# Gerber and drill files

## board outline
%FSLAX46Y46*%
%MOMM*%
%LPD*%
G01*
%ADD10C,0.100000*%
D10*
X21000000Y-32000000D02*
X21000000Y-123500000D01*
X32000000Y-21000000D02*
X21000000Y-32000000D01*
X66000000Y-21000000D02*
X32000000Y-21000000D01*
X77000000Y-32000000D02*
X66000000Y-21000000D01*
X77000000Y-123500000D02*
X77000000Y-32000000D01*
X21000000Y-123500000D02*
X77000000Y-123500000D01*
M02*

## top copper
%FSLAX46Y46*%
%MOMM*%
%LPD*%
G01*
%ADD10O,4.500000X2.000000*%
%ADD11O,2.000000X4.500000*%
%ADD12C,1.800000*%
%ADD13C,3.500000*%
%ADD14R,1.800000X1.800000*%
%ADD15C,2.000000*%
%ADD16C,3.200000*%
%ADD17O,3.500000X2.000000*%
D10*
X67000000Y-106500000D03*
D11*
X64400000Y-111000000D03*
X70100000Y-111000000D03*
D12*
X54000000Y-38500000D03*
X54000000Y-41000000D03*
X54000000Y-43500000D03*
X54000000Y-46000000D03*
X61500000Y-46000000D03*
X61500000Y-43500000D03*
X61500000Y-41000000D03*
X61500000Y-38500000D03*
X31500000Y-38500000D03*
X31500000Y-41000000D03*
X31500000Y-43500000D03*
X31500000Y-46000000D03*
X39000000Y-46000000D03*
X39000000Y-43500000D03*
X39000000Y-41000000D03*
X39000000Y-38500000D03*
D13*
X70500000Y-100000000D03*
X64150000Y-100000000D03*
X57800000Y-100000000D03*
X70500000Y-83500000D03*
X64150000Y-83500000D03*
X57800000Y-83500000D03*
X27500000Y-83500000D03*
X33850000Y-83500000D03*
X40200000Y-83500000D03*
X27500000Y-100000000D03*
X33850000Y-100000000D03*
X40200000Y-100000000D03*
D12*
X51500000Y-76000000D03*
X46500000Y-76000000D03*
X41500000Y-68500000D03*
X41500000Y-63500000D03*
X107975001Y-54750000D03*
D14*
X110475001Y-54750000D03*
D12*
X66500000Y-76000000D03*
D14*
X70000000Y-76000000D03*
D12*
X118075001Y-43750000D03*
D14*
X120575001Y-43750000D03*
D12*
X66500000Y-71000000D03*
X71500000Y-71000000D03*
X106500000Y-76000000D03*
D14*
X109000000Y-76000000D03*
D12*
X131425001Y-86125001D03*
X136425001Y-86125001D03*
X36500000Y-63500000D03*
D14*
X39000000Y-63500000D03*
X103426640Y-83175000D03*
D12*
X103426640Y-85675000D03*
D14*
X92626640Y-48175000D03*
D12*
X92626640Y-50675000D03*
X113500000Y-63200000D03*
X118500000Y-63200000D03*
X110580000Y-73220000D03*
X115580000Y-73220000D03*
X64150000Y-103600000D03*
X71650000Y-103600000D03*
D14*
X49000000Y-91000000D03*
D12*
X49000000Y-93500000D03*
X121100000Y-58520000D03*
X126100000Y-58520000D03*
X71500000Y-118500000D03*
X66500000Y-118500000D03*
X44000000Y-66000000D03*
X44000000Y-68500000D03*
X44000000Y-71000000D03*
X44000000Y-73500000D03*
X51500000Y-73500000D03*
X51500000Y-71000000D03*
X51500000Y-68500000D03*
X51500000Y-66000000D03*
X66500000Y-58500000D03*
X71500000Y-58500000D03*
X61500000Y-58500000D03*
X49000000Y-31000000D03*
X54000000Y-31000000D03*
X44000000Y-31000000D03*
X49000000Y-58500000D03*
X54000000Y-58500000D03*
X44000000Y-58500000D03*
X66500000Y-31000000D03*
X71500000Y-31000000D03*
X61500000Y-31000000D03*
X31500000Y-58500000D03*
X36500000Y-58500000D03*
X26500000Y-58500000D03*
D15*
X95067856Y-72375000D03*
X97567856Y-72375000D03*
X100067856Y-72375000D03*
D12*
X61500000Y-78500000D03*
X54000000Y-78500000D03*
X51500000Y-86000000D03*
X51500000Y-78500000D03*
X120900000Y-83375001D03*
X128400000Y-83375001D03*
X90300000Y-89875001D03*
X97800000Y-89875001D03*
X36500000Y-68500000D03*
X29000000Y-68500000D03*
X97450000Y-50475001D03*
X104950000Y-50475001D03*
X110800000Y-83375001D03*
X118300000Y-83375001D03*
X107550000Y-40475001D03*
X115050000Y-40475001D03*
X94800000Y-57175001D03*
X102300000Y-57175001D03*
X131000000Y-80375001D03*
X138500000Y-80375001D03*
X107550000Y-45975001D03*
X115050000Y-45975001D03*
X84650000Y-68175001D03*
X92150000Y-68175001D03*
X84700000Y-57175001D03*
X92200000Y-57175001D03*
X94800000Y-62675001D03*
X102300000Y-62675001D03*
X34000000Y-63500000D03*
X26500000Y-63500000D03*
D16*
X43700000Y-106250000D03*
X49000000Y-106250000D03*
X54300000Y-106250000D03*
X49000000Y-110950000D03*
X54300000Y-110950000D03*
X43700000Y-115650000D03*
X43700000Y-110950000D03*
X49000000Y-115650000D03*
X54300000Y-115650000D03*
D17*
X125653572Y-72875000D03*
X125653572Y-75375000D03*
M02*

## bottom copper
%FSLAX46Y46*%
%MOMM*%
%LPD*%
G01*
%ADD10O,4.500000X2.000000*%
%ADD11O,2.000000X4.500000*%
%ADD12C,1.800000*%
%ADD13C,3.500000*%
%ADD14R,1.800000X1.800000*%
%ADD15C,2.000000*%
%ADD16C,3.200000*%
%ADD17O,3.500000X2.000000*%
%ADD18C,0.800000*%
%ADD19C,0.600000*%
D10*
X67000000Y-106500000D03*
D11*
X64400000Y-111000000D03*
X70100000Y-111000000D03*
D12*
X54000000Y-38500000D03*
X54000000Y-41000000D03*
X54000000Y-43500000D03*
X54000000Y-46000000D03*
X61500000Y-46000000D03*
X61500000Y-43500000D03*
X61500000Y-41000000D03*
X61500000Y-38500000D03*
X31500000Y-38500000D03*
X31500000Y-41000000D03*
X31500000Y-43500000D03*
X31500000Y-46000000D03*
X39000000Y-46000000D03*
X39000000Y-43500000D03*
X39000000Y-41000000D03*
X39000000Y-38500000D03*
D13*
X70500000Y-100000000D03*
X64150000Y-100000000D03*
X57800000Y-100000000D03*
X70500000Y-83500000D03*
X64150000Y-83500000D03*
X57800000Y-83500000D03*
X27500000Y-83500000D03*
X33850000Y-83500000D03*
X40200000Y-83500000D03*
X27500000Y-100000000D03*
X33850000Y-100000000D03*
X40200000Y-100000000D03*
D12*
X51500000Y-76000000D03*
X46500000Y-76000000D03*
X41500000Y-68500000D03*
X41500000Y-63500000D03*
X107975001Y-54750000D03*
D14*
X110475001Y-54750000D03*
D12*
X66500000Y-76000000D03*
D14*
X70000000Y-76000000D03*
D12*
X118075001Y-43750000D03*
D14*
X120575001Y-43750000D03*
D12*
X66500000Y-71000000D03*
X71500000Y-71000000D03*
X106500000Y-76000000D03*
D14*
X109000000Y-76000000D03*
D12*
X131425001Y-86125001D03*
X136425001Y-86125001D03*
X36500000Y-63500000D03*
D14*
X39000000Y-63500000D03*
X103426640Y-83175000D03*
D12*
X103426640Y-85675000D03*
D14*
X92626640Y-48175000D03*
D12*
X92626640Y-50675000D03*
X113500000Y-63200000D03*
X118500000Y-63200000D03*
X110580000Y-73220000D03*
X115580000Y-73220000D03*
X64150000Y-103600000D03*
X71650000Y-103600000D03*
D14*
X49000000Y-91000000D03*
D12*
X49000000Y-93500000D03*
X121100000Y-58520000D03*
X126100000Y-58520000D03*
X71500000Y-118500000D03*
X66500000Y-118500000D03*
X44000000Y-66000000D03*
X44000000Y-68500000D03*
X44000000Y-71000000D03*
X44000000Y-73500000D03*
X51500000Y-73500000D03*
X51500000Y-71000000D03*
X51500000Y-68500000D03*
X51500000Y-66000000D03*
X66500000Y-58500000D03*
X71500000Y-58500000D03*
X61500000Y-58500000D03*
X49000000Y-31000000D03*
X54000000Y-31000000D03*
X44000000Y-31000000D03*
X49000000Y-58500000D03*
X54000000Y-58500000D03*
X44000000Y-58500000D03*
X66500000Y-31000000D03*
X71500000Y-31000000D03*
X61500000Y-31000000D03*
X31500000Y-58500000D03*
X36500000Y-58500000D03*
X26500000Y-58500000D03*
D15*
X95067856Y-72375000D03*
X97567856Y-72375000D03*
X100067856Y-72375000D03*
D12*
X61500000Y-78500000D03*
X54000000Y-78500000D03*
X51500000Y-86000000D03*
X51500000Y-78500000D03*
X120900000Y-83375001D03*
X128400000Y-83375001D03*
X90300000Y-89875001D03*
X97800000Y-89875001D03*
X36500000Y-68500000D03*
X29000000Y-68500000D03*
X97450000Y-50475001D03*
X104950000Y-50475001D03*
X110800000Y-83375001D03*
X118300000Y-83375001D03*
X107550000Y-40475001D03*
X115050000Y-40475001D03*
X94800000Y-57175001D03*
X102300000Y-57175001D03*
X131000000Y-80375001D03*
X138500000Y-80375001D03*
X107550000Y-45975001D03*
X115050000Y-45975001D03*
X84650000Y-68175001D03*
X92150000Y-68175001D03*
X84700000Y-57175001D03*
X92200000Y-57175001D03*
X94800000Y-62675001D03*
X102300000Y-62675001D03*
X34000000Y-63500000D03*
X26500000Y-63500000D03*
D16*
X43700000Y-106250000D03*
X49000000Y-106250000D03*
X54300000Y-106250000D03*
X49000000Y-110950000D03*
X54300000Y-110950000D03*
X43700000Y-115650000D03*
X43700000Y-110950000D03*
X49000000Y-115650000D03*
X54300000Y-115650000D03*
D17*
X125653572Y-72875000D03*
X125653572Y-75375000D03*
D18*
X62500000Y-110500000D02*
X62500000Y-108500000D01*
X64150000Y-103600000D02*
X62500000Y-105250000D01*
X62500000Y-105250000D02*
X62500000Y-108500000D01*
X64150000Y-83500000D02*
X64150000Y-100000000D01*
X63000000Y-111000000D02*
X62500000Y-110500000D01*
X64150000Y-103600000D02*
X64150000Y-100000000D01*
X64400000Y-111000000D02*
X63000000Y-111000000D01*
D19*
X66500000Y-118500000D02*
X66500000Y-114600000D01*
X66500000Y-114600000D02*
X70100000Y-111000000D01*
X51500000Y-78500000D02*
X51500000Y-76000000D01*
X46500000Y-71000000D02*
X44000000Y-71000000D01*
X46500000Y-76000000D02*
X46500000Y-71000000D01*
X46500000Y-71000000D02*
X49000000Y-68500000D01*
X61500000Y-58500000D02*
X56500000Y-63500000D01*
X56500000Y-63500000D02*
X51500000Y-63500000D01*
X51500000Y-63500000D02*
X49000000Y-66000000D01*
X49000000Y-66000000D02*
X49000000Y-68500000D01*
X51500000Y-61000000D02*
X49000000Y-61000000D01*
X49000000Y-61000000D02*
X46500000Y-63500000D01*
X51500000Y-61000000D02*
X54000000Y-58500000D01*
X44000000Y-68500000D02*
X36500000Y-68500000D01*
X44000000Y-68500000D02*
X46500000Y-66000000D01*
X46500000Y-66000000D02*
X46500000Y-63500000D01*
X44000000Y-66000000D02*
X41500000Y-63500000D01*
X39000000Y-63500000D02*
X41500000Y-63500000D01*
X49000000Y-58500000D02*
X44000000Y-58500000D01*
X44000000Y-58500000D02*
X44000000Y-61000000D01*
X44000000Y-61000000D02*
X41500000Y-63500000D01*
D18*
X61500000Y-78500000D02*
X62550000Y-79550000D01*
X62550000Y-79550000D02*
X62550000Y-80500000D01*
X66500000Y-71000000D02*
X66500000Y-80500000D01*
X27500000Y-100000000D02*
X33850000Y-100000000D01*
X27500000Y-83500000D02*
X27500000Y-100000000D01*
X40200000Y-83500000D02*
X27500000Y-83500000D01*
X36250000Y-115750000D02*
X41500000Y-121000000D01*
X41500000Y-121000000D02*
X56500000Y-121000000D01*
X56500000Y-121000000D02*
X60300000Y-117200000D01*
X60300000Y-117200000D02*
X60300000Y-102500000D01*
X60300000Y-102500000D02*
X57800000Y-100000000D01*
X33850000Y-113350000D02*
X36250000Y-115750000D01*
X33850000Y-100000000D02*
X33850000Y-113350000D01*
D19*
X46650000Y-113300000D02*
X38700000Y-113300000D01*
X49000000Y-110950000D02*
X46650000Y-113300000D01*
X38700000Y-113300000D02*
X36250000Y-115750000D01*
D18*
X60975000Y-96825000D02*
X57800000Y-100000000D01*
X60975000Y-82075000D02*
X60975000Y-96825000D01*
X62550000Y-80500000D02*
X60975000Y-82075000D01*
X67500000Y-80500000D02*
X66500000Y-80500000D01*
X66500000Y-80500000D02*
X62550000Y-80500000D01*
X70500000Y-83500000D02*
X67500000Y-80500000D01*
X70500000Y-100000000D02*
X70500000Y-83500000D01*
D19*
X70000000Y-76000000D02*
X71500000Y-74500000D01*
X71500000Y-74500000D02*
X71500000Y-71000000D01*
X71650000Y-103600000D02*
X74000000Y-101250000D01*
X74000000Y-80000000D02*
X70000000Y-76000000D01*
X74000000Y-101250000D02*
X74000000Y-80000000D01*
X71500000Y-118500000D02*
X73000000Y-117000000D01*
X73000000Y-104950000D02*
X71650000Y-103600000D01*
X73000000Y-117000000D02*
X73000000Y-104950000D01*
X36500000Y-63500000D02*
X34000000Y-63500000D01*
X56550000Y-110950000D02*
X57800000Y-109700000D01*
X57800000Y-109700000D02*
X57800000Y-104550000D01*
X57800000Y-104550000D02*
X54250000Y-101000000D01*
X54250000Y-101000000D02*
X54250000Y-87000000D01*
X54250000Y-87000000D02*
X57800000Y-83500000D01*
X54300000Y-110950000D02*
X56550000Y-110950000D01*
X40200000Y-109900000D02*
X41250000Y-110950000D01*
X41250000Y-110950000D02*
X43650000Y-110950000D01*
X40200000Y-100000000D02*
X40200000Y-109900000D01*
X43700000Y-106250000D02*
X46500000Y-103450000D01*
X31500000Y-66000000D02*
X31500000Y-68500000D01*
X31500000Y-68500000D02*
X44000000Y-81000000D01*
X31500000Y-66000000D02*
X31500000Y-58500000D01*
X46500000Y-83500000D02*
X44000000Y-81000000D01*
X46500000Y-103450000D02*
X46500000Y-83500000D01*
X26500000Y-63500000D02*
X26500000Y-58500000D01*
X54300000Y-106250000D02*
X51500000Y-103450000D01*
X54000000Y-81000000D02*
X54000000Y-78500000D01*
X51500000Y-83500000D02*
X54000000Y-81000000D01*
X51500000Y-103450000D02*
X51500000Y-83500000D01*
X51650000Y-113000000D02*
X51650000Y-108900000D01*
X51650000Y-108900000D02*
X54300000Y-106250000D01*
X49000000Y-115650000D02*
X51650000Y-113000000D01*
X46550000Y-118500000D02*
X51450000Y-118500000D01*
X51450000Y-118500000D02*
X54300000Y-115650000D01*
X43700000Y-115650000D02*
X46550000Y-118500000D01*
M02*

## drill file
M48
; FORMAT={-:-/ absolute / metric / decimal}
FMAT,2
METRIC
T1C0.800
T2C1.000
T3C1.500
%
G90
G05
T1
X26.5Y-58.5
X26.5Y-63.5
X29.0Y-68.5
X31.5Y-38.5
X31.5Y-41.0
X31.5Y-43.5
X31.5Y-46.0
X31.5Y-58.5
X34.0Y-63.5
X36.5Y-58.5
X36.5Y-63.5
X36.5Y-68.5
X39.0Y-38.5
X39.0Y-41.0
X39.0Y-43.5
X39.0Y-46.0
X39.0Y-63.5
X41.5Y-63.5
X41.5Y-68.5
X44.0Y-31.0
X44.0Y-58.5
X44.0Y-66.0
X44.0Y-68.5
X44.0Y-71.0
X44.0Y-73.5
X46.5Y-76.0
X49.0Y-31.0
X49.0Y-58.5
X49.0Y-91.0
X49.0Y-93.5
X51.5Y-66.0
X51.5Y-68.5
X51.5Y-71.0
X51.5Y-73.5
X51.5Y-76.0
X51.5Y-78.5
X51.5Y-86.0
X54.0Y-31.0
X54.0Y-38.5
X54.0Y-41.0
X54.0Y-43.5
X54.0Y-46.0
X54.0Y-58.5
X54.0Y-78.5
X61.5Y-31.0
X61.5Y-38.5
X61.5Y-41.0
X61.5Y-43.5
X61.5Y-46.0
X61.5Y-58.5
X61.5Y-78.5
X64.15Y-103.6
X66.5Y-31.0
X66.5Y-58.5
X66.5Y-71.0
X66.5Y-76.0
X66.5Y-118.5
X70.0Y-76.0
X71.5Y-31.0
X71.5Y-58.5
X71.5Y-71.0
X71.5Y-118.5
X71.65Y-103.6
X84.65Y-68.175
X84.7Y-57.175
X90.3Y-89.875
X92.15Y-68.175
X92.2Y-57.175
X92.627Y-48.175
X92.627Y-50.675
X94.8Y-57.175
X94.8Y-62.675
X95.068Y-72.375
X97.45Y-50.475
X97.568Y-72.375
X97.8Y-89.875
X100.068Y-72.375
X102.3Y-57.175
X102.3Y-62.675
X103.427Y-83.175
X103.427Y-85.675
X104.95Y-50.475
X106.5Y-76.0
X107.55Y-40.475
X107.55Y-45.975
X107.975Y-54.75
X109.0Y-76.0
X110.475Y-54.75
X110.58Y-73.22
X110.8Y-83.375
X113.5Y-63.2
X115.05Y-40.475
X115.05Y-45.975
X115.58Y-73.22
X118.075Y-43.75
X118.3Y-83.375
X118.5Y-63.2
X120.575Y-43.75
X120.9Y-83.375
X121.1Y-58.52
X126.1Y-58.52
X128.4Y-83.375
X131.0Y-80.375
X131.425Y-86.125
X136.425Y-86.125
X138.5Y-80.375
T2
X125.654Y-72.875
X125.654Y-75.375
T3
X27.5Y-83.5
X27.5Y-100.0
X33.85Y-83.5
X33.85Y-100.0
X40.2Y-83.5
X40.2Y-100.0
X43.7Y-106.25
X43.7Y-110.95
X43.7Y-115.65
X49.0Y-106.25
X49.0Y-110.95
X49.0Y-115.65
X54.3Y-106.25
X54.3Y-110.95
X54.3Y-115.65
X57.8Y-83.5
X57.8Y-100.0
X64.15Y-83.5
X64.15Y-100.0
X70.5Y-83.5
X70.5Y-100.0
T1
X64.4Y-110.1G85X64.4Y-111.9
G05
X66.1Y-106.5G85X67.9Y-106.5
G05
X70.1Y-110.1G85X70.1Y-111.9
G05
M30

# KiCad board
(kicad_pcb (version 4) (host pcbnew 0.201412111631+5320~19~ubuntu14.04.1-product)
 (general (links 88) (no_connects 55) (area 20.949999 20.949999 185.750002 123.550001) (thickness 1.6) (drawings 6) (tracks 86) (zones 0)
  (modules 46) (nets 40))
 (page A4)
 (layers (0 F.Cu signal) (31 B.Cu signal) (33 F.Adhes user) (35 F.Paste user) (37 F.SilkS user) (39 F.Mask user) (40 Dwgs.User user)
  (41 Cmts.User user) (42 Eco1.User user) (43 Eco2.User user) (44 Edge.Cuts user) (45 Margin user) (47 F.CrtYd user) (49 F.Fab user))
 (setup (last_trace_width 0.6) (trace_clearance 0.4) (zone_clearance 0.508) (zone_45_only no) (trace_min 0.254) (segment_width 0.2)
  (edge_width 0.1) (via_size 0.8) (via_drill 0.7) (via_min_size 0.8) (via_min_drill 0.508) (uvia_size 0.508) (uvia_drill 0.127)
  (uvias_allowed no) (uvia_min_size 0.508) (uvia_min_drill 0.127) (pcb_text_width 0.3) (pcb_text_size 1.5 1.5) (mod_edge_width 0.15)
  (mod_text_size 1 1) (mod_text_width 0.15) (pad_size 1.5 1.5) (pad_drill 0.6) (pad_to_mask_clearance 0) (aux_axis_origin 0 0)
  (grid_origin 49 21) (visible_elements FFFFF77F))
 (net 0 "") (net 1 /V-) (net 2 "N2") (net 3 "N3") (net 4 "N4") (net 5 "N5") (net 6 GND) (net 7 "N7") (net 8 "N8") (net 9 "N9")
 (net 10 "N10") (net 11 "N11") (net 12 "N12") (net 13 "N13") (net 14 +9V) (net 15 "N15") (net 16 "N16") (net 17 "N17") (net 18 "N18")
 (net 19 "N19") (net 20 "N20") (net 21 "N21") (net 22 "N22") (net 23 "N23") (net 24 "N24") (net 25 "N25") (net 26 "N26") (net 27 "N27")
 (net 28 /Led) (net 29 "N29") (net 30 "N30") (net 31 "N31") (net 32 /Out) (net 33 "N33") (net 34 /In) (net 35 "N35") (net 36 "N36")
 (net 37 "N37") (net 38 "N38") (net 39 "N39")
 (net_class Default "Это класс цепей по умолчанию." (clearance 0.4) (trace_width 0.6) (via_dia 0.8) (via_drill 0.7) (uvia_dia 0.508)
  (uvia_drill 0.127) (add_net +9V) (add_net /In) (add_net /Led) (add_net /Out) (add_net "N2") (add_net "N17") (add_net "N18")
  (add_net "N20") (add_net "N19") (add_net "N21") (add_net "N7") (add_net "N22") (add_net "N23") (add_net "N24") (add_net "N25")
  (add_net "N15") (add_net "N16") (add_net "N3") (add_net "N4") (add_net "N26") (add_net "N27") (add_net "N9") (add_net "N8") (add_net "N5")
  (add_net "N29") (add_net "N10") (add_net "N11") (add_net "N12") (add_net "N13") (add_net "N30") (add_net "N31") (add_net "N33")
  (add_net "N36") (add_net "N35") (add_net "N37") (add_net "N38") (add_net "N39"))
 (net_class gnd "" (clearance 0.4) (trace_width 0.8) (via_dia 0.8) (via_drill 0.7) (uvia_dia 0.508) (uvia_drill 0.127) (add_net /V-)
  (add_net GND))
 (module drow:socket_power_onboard (layer F.Cu) (at 67 106.5)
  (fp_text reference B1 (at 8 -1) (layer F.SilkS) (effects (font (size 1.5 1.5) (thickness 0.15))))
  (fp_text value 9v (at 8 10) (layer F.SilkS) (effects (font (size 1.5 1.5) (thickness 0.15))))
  (pad 3 thru_hole oval (at 0 0) (size 4.5 2) (drill oval 2.6 0.8) (layers *.Cu *.Mask))
  (pad 2 thru_hole oval (at -2.6 4.5) (size 2 4.5) (drill oval 0.8 2.6) (layers *.Cu *.Mask) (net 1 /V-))
  (pad 1 thru_hole oval (at 3.1 4.5) (size 2 4.5) (drill oval 0.8 2.6) (layers *.Cu *.Mask) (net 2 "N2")))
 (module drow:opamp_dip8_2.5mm (layer F.Cu) (at 54 38.5)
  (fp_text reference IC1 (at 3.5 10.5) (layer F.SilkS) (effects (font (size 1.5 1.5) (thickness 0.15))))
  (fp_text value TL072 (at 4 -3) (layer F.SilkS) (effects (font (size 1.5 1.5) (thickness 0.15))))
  (pad 1 thru_hole circle (at 0 0) (size 1.8 1.8) (drill 0.8) (layers *.Cu *.Mask) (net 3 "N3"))
  (pad 2 thru_hole circle (at 0 2.5) (size 1.8 1.8) (drill 0.8) (layers *.Cu *.Mask) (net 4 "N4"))
  (pad 3 thru_hole circle (at 0 5) (size 1.8 1.8) (drill 0.8) (layers *.Cu *.Mask) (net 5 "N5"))
  (pad 4 thru_hole circle (at 0 7.5) (size 1.8 1.8) (drill 0.8) (layers *.Cu *.Mask) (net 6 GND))
  (pad 5 thru_hole circle (at 7.5 7.5) (size 1.8 1.8) (drill 0.8) (layers *.Cu *.Mask) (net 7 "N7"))
  (pad 6 thru_hole circle (at 7.5 5) (size 1.8 1.8) (drill 0.8) (layers *.Cu *.Mask) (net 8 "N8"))
  (pad 7 thru_hole circle (at 7.5 2.5) (size 1.8 1.8) (drill 0.8) (layers *.Cu *.Mask) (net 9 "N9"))
  (pad 8 thru_hole circle (at 7.5 0) (size 1.8 1.8) (drill 0.8) (layers *.Cu *.Mask)))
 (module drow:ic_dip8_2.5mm (layer F.Cu) (at 31.5 38.5)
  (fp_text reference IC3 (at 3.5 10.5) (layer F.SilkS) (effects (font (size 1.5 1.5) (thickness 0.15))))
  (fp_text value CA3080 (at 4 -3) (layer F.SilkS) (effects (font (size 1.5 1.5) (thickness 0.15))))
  (pad 1 thru_hole circle (at 0 0) (size 1.8 1.8) (drill 0.8) (layers *.Cu *.Mask))
  (pad 2 thru_hole circle (at 0 2.5) (size 1.8 1.8) (drill 0.8) (layers *.Cu *.Mask) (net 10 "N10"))
  (pad 3 thru_hole circle (at 0 5) (size 1.8 1.8) (drill 0.8) (layers *.Cu *.Mask) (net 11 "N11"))
  (pad 4 thru_hole circle (at 0 7.5) (size 1.8 1.8) (drill 0.8) (layers *.Cu *.Mask) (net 6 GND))
  (pad 5 thru_hole circle (at 7.5 7.5) (size 1.8 1.8) (drill 0.8) (layers *.Cu *.Mask) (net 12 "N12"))
  (pad 6 thru_hole circle (at 7.5 5) (size 1.8 1.8) (drill 0.8) (layers *.Cu *.Mask) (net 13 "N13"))
  (pad 7 thru_hole circle (at 7.5 2.5) (size 1.8 1.8) (drill 0.8) (layers *.Cu *.Mask) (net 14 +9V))
  (pad 8 thru_hole circle (at 7.5 0) (size 1.8 1.8) (drill 0.8) (layers *.Cu *.Mask)))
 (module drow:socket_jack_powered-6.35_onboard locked (layer F.Cu) (at 70.5 100 180)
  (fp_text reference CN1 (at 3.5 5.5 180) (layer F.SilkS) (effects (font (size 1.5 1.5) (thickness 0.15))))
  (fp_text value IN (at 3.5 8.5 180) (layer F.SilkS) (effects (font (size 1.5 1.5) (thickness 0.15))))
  (pad 2 thru_hole circle (at 0 0 180) (size 3.5 3.5) (drill 1.5) (layers *.Cu *.Mask F.SilkS) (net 6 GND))
  (pad 3 thru_hole circle (at 6.35 0 180) (size 3.5 3.5) (drill 1.5) (layers *.Cu *.Mask F.SilkS) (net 1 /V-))
  (pad 2 thru_hole circle (at 12.7 0 180) (size 3.5 3.5) (drill 1.5) (layers *.Cu *.Mask F.SilkS) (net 6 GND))
  (pad 2 thru_hole circle (at 0 16.5 180) (size 3.5 3.5) (drill 1.5) (layers *.Cu *.Mask F.SilkS) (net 6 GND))
  (pad 3 thru_hole circle (at 6.35 16.5 180) (size 3.5 3.5) (drill 1.5) (layers *.Cu *.Mask F.SilkS) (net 1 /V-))
  (pad 1 thru_hole circle (at 12.7 16.5 180) (size 3.5 3.5) (drill 1.5) (layers *.Cu *.Mask F.SilkS) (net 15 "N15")))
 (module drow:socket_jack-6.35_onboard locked (layer F.Cu) (at 27.5 83.5)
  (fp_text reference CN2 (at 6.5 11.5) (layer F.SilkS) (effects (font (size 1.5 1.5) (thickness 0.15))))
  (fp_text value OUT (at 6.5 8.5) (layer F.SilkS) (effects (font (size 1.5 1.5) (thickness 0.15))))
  (pad 2 thru_hole circle (at 0 0) (size 3.5 3.5) (drill 1.5) (layers *.Cu *.Mask F.SilkS) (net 6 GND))
  (pad 2 thru_hole circle (at 6.35 0) (size 3.5 3.5) (drill 1.5) (layers *.Cu *.Mask F.SilkS) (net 6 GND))
  (pad 2 thru_hole circle (at 12.7 0) (size 3.5 3.5) (drill 1.5) (layers *.Cu *.Mask F.SilkS) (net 6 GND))
  (pad 2 thru_hole circle (at 0 16.5) (size 3.5 3.5) (drill 1.5) (layers *.Cu *.Mask F.SilkS) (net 6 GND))
  (pad 2 thru_hole circle (at 6.35 16.5) (size 3.5 3.5) (drill 1.5) (layers *.Cu *.Mask F.SilkS) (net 6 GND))
  (pad 1 thru_hole circle (at 12.7 16.5) (size 3.5 3.5) (drill 1.5) (layers *.Cu *.Mask F.SilkS) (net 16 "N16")))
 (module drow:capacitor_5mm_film (layer F.Cu) (at 51.5 76 180)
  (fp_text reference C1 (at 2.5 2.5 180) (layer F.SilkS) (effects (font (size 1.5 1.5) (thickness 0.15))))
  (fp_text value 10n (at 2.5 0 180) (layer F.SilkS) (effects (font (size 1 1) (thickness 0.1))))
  (pad 1 thru_hole circle (at 0 0 180) (size 1.8 1.8) (drill 0.8) (layers *.Cu *.Mask F.SilkS) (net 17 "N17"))
  (pad 2 thru_hole circle (at 5 0 180) (size 1.8 1.8) (drill 0.8) (layers *.Cu *.Mask F.SilkS) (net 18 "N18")))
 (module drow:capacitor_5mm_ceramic (layer F.Cu) (at 41.5 63.5 270)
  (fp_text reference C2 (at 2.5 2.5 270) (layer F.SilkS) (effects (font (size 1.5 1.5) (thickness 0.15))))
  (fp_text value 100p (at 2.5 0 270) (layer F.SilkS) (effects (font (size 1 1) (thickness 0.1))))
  (pad 2 thru_hole circle (at 5 0 270) (size 1.8 1.8) (drill 0.8) (layers *.Cu *.Mask F.SilkS) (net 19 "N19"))
  (pad 1 thru_hole circle (at 0 0 270) (size 1.8 1.8) (drill 0.8) (layers *.Cu *.Mask F.SilkS) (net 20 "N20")))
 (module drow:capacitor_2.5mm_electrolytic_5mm (layer F.Cu) (at 107.975001 54.75)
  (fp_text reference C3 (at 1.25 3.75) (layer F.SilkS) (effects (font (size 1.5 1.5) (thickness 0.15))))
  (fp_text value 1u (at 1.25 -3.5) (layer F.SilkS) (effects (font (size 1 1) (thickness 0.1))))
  (pad 1 thru_hole circle (at 0 0) (size 1.8 1.8) (drill 0.8) (layers *.Cu *.Mask F.SilkS) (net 6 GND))
  (pad 2 thru_hole rect (at 2.5 0) (size 1.8 1.8) (drill 0.8) (layers *.Cu *.Mask F.SilkS) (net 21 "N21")))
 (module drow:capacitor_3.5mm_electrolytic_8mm (layer F.Cu) (at 66.5 76)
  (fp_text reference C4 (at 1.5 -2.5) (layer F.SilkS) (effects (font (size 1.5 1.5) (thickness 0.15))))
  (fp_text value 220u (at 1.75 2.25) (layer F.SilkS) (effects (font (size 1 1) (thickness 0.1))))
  (pad 1 thru_hole circle (at 0 0) (size 1.8 1.8) (drill 0.8) (layers *.Cu *.Mask F.SilkS) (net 6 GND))
  (pad 2 thru_hole rect (at 3.5 0) (size 1.8 1.8) (drill 0.8) (layers *.Cu *.Mask F.SilkS) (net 14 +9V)))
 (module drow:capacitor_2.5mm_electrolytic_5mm (layer F.Cu) (at 118.075001 43.75)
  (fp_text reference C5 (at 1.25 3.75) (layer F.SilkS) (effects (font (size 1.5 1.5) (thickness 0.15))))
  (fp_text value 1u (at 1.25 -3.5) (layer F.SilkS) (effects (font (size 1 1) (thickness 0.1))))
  (pad 1 thru_hole circle (at 0 0) (size 1.8 1.8) (drill 0.8) (layers *.Cu *.Mask F.SilkS) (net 6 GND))
  (pad 2 thru_hole rect (at 2.5 0) (size 1.8 1.8) (drill 0.8) (layers *.Cu *.Mask F.SilkS) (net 7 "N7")))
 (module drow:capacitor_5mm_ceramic (layer F.Cu) (at 71.5 71 180)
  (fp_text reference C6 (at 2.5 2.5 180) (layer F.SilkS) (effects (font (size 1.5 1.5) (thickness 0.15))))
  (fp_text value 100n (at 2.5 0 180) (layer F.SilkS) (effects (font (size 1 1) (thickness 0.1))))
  (pad 2 thru_hole circle (at 5 0 180) (size 1.8 1.8) (drill 0.8) (layers *.Cu *.Mask F.SilkS) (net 6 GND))
  (pad 1 thru_hole circle (at 0 0 180) (size 1.8 1.8) (drill 0.8) (layers *.Cu *.Mask F.SilkS) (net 14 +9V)))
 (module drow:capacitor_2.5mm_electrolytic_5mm (layer F.Cu) (at 106.5 76)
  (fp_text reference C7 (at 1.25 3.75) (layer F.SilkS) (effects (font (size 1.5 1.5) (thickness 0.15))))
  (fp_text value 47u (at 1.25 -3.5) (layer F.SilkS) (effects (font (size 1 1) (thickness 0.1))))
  (pad 1 thru_hole circle (at 0 0) (size 1.8 1.8) (drill 0.8) (layers *.Cu *.Mask F.SilkS) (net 6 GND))
  (pad 2 thru_hole rect (at 2.5 0) (size 1.8 1.8) (drill 0.8) (layers *.Cu *.Mask F.SilkS) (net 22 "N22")))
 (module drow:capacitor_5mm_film (layer F.Cu) (at 131.425001 86.125001)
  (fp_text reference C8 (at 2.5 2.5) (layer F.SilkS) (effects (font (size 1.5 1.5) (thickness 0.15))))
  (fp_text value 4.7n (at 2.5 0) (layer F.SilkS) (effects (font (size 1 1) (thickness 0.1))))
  (pad 1 thru_hole circle (at 0 0) (size 1.8 1.8) (drill 0.8) (layers *.Cu *.Mask F.SilkS) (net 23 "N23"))
  (pad 2 thru_hole circle (at 5 0) (size 1.8 1.8) (drill 0.8) (layers *.Cu *.Mask F.SilkS) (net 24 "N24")))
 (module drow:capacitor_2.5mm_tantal (layer F.Cu) (at 36.5 63.5)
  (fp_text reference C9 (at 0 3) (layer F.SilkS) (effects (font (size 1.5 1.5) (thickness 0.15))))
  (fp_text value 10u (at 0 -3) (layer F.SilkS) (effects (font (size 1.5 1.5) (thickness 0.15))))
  (pad 1 thru_hole circle (at 0 0) (size 1.8 1.8) (drill 0.8) (layers *.Cu *.Mask F.SilkS) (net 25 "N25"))
  (pad 2 thru_hole rect (at 2.5 0) (size 1.8 1.8) (drill 0.8) (layers *.Cu *.Mask F.SilkS) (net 20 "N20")))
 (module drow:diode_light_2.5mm (layer F.Cu) (at 103.42664 83.175)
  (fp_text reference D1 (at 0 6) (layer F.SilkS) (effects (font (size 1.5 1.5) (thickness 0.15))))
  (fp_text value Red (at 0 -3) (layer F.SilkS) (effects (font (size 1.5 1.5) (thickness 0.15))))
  (pad 1 thru_hole rect (at 0 0) (size 1.8 1.8) (drill 0.8) (layers *.Cu *.Mask F.SilkS) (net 17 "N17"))
  (pad 2 thru_hole circle (at 0 2.5) (size 1.8 1.8) (drill 0.8) (layers *.Cu *.Mask F.SilkS) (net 6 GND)))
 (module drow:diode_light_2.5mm (layer F.Cu) (at 92.62664 48.175)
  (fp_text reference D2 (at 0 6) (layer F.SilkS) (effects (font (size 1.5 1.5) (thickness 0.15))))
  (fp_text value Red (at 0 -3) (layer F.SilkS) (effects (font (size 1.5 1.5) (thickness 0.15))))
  (pad 1 thru_hole rect (at 0 0) (size 1.8 1.8) (drill 0.8) (layers *.Cu *.Mask F.SilkS) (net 6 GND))
  (pad 2 thru_hole circle (at 0 2.5) (size 1.8 1.8) (drill 0.8) (layers *.Cu *.Mask F.SilkS) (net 17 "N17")))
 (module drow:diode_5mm (layer F.Cu) (at 113.5 63.2)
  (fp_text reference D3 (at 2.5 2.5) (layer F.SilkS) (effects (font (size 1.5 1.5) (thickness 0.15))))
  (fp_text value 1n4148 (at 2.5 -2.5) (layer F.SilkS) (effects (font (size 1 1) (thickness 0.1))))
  (pad 1 thru_hole circle (at 0 0) (size 1.8 1.8) (drill 0.8) (layers *.Cu *.Mask F.SilkS) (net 3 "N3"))
  (pad 2 thru_hole circle (at 5 0) (size 1.8 1.8) (drill 0.8) (layers *.Cu *.Mask F.SilkS) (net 4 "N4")))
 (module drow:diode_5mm (layer F.Cu) (at 110.58 73.22)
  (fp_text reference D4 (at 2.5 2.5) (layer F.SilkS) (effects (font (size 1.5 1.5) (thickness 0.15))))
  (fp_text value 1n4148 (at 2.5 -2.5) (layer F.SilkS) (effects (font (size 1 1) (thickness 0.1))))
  (pad 1 thru_hole circle (at 0 0) (size 1.8 1.8) (drill 0.8) (layers *.Cu *.Mask F.SilkS) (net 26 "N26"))
  (pad 2 thru_hole circle (at 5 0) (size 1.8 1.8) (drill 0.8) (layers *.Cu *.Mask F.SilkS) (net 3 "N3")))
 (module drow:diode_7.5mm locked (layer F.Cu) (at 64.15 103.6)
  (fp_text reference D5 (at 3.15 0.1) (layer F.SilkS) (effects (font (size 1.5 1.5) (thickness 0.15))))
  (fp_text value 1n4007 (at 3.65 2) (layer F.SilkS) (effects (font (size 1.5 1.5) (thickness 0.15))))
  (pad 1 thru_hole circle (at 0 0) (size 1.8 1.8) (drill 0.8) (layers *.Cu *.Mask F.SilkS) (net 1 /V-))
  (pad 2 thru_hole circle (at 7.5 0) (size 1.8 1.8) (drill 0.8) (layers *.Cu *.Mask F.SilkS) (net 14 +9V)))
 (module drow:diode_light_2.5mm (layer F.Cu) (at 49 91)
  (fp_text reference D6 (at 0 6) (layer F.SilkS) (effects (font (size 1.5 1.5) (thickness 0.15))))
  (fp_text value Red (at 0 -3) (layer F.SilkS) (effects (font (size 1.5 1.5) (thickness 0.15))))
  (pad 1 thru_hole rect (at 0 0) (size 1.8 1.8) (drill 0.8) (layers *.Cu *.Mask F.SilkS) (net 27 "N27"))
  (pad 2 thru_hole circle (at 0 2.5) (size 1.8 1.8) (drill 0.8) (layers *.Cu *.Mask F.SilkS) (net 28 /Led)))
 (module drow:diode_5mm (layer F.Cu) (at 121.1 58.52)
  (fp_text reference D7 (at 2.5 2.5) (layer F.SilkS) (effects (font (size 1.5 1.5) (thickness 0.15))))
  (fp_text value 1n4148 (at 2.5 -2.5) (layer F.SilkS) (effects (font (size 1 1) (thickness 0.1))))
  (pad 1 thru_hole circle (at 0 0) (size 1.8 1.8) (drill 0.8) (layers *.Cu *.Mask F.SilkS) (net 9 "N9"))
  (pad 2 thru_hole circle (at 5 0) (size 1.8 1.8) (drill 0.8) (layers *.Cu *.Mask F.SilkS) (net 8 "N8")))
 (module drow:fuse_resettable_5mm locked (layer F.Cu) (at 71.5 118.5 180)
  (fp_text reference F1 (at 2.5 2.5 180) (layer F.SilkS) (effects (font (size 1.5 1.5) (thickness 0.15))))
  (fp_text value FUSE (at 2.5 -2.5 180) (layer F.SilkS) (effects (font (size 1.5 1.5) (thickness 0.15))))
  (pad 1 thru_hole circle (at 0 0 180) (size 1.8 1.8) (drill 0.8) (layers *.Cu *.Mask F.SilkS) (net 14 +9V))
  (pad 2 thru_hole circle (at 5 0 180) (size 1.8 1.8) (drill 0.8) (layers *.Cu *.Mask F.SilkS) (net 2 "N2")))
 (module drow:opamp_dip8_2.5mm (layer F.Cu) (at 44 66)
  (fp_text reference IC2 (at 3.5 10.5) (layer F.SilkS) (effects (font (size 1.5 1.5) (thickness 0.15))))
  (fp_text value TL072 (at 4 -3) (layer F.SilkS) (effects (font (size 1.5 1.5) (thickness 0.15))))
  (pad 1 thru_hole circle (at 0 0) (size 1.8 1.8) (drill 0.8) (layers *.Cu *.Mask F.SilkS) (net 20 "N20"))
  (pad 2 thru_hole circle (at 0 2.5) (size 1.8 1.8) (drill 0.8) (layers *.Cu *.Mask F.SilkS) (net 19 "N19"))
  (pad 3 thru_hole circle (at 0 5) (size 1.8 1.8) (drill 0.8) (layers *.Cu *.Mask F.SilkS) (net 18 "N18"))
  (pad 4 thru_hole circle (at 0 7.5) (size 1.8 1.8) (drill 0.8) (layers *.Cu *.Mask F.SilkS) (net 6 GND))
  (pad 5 thru_hole circle (at 7.5 7.5) (size 1.8 1.8) (drill 0.8) (layers *.Cu *.Mask F.SilkS) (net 22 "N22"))
  (pad 6 thru_hole circle (at 7.5 5) (size 1.8 1.8) (drill 0.8) (layers *.Cu *.Mask F.SilkS) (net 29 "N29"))
  (pad 7 thru_hole circle (at 7.5 2.5) (size 1.8 1.8) (drill 0.8) (layers *.Cu *.Mask F.SilkS) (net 14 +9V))
  (pad 8 thru_hole circle (at 7.5 0) (size 1.8 1.8) (drill 0.8) (layers *.Cu *.Mask F.SilkS)))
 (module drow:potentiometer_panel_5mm (layer F.Cu) (at 66.5 58.5)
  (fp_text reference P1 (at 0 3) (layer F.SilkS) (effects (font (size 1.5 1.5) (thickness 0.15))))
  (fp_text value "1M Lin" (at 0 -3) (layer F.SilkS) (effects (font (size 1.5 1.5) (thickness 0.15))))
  (pad 2 thru_hole circle (at 0 0) (size 1.8 1.8) (drill 0.8) (layers *.Cu *.Mask F.SilkS) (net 5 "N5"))
  (pad 1 thru_hole circle (at 5 0) (size 1.8 1.8) (drill 0.8) (layers *.Cu *.Mask F.SilkS) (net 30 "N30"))
  (pad 3 thru_hole circle (at -5 0) (size 1.8 1.8) (drill 0.8) (layers *.Cu *.Mask F.SilkS) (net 18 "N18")))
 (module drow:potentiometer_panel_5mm (layer F.Cu) (at 49 31)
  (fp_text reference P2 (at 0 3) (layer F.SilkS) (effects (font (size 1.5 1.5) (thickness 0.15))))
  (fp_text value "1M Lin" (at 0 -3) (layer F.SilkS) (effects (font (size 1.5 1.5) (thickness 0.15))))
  (pad 2 thru_hole circle (at 0 0) (size 1.8 1.8) (drill 0.8) (layers *.Cu *.Mask F.SilkS) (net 4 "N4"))
  (pad 1 thru_hole circle (at 5 0) (size 1.8 1.8) (drill 0.8) (layers *.Cu *.Mask F.SilkS) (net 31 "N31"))
  (pad 3 thru_hole circle (at -5 0) (size 1.8 1.8) (drill 0.8) (layers *.Cu *.Mask F.SilkS) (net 4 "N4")))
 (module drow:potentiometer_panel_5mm (layer F.Cu) (at 49 58.5)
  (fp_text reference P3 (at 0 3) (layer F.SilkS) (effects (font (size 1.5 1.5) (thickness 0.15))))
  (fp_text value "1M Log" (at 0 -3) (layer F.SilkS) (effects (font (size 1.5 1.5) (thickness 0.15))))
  (pad 2 thru_hole circle (at 0 0) (size 1.8 1.8) (drill 0.8) (layers *.Cu *.Mask F.SilkS) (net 20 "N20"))
  (pad 1 thru_hole circle (at 5 0) (size 1.8 1.8) (drill 0.8) (layers *.Cu *.Mask F.SilkS) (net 19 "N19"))
  (pad 3 thru_hole circle (at -5 0) (size 1.8 1.8) (drill 0.8) (layers *.Cu *.Mask F.SilkS) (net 20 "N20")))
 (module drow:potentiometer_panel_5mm (layer F.Cu) (at 66.5 31)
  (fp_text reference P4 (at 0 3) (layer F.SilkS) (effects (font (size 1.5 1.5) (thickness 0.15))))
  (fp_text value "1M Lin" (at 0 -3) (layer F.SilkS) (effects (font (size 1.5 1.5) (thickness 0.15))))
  (pad 2 thru_hole circle (at 0 0) (size 1.8 1.8) (drill 0.8) (layers *.Cu *.Mask F.SilkS) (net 26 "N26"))
  (pad 1 thru_hole circle (at 5 0) (size 1.8 1.8) (drill 0.8) (layers *.Cu *.Mask F.SilkS) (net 21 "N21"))
  (pad 3 thru_hole circle (at -5 0) (size 1.8 1.8) (drill 0.8) (layers *.Cu *.Mask F.SilkS) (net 26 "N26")))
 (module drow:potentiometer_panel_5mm (layer F.Cu) (at 31.5 58.5)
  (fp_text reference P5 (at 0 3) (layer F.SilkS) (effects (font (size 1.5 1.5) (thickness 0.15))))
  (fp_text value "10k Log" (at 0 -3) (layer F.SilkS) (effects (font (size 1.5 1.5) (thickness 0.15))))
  (pad 2 thru_hole circle (at 0 0) (size 1.8 1.8) (drill 0.8) (layers *.Cu *.Mask F.SilkS) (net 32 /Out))
  (pad 1 thru_hole circle (at 5 0) (size 1.8 1.8) (drill 0.8) (layers *.Cu *.Mask F.SilkS) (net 6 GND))
  (pad 3 thru_hole circle (at -5 0) (size 1.8 1.8) (drill 0.8) (layers *.Cu *.Mask F.SilkS) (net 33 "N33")))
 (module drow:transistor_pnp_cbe (layer F.Cu) (at 97.567856 72.375)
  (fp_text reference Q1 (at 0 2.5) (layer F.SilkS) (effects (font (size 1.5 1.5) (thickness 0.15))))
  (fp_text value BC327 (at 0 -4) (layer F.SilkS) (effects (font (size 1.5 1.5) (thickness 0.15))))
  (pad 1 thru_hole circle (at -2.5 0) (size 2 2) (drill 0.8) (layers *.Cu *.Mask F.SilkS) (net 12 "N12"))
  (pad 2 thru_hole circle (at 0 0) (size 2 2) (drill 0.8) (layers *.Cu *.Mask F.SilkS) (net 9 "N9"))
  (pad 3 thru_hole circle (at 2.5 0) (size 2 2) (drill 0.8) (layers *.Cu *.Mask F.SilkS) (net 8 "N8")))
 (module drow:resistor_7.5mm (layer F.Cu) (at 61.5 78.5 180)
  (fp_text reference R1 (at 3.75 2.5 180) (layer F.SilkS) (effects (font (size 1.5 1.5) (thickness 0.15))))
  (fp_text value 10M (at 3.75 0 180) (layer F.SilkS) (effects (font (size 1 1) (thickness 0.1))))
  (pad 1 thru_hole circle (at 0 0 180) (size 1.8 1.8) (drill 0.8) (layers *.Cu *.Mask F.SilkS) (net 6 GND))
  (pad 2 thru_hole circle (at 7.5 0 180) (size 1.8 1.8) (drill 0.8) (layers *.Cu *.Mask F.SilkS) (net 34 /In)))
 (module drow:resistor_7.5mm (layer F.Cu) (at 51.5 86 90)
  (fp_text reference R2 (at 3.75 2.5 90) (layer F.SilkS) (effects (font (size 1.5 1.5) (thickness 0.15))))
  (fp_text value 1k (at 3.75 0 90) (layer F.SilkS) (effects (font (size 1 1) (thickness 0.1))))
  (pad 1 thru_hole circle (at 0 0 90) (size 1.8 1.8) (drill 0.8) (layers *.Cu *.Mask F.SilkS) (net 34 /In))
  (pad 2 thru_hole circle (at 7.5 0 90) (size 1.8 1.8) (drill 0.8) (layers *.Cu *.Mask F.SilkS) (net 17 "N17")))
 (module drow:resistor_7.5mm (layer F.Cu) (at 120.9 83.375001)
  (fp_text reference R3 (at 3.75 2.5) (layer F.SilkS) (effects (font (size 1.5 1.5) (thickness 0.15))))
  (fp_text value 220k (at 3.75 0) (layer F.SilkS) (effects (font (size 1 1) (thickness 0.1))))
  (pad 1 thru_hole circle (at 0 0) (size 1.8 1.8) (drill 0.8) (layers *.Cu *.Mask F.SilkS) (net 31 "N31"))
  (pad 2 thru_hole circle (at 7.5 0) (size 1.8 1.8) (drill 0.8) (layers *.Cu *.Mask F.SilkS) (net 21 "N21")))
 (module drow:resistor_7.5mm (layer F.Cu) (at 90.3 89.875001)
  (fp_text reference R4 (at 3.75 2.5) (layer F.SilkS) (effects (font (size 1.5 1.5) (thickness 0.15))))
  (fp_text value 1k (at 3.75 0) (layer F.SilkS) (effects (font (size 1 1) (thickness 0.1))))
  (pad 1 thru_hole circle (at 0 0) (size 1.8 1.8) (drill 0.8) (layers *.Cu *.Mask F.SilkS) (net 21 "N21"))
  (pad 2 thru_hole circle (at 7.5 0) (size 1.8 1.8) (drill 0.8) (layers *.Cu *.Mask F.SilkS) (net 7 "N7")))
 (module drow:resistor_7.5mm (layer F.Cu) (at 36.5 68.5 180)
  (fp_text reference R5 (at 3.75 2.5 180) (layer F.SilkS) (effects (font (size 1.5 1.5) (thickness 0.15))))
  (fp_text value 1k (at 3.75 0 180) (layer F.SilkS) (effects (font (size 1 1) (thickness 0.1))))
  (pad 1 thru_hole circle (at 0 0 180) (size 1.8 1.8) (drill 0.8) (layers *.Cu *.Mask F.SilkS) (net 19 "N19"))
  (pad 2 thru_hole circle (at 7.5 0 180) (size 1.8 1.8) (drill 0.8) (layers *.Cu *.Mask F.SilkS) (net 13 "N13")))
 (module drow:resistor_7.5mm (layer F.Cu) (at 97.45 50.475001)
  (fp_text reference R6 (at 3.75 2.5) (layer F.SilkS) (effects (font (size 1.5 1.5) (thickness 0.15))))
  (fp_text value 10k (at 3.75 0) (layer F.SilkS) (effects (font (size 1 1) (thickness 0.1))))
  (pad 1 thru_hole circle (at 0 0) (size 1.8 1.8) (drill 0.8) (layers *.Cu *.Mask F.SilkS) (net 14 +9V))
  (pad 2 thru_hole circle (at 7.5 0) (size 1.8 1.8) (drill 0.8) (layers *.Cu *.Mask F.SilkS) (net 27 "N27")))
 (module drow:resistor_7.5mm (layer F.Cu) (at 110.8 83.375001)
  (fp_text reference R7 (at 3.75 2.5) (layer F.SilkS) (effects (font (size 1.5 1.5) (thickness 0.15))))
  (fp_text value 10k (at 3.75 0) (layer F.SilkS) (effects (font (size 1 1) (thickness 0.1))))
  (pad 1 thru_hole circle (at 0 0) (size 1.8 1.8) (drill 0.8) (layers *.Cu *.Mask F.SilkS) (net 14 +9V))
  (pad 2 thru_hole circle (at 7.5 0) (size 1.8 1.8) (drill 0.8) (layers *.Cu *.Mask F.SilkS) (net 22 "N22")))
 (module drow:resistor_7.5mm (layer F.Cu) (at 107.55 40.475001)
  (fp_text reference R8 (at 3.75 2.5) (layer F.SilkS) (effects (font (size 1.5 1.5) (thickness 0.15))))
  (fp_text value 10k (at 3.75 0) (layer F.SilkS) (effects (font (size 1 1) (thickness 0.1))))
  (pad 1 thru_hole circle (at 0 0) (size 1.8 1.8) (drill 0.8) (layers *.Cu *.Mask F.SilkS) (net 22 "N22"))
  (pad 2 thru_hole circle (at 7.5 0) (size 1.8 1.8) (drill 0.8) (layers *.Cu *.Mask F.SilkS) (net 6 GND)))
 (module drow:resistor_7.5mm (layer F.Cu) (at 94.8 57.175001)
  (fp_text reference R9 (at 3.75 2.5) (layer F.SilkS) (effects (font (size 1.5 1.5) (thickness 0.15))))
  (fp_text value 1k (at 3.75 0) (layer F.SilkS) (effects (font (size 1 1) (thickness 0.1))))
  (pad 1 thru_hole circle (at 0 0) (size 1.8 1.8) (drill 0.8) (layers *.Cu *.Mask F.SilkS) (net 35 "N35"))
  (pad 2 thru_hole circle (at 7.5 0) (size 1.8 1.8) (drill 0.8) (layers *.Cu *.Mask F.SilkS) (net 8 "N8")))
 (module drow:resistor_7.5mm (layer F.Cu) (at 131 80.375001)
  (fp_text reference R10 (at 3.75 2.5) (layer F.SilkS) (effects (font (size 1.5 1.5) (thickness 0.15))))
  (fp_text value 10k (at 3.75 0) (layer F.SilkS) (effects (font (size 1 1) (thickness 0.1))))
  (pad 1 thru_hole circle (at 0 0) (size 1.8 1.8) (drill 0.8) (layers *.Cu *.Mask F.SilkS) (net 13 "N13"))
  (pad 2 thru_hole circle (at 7.5 0) (size 1.8 1.8) (drill 0.8) (layers *.Cu *.Mask F.SilkS) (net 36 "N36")))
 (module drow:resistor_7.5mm (layer F.Cu) (at 107.55 45.975001)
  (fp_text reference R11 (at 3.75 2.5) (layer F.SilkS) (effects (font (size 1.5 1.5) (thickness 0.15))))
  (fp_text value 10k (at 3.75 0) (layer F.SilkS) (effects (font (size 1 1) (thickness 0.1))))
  (pad 1 thru_hole circle (at 0 0) (size 1.8 1.8) (drill 0.8) (layers *.Cu *.Mask F.SilkS) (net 13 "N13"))
  (pad 2 thru_hole circle (at 7.5 0) (size 1.8 1.8) (drill 0.8) (layers *.Cu *.Mask F.SilkS) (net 23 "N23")))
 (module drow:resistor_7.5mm (layer F.Cu) (at 84.65 68.175001)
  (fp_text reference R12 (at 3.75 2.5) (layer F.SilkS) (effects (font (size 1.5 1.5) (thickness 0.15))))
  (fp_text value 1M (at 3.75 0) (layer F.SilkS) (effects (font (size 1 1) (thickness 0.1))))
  (pad 1 thru_hole circle (at 0 0) (size 1.8 1.8) (drill 0.8) (layers *.Cu *.Mask F.SilkS) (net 12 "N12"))
  (pad 2 thru_hole circle (at 7.5 0) (size 1.8 1.8) (drill 0.8) (layers *.Cu *.Mask F.SilkS) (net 35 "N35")))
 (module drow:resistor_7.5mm (layer F.Cu) (at 84.7 57.175001)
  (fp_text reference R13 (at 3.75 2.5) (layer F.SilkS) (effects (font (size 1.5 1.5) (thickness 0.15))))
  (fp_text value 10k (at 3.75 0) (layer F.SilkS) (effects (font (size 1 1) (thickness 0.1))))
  (pad 1 thru_hole circle (at 0 0) (size 1.8 1.8) (drill 0.8) (layers *.Cu *.Mask F.SilkS) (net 11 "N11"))
  (pad 2 thru_hole circle (at 7.5 0) (size 1.8 1.8) (drill 0.8) (layers *.Cu *.Mask F.SilkS) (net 20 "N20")))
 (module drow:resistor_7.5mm (layer F.Cu) (at 94.8 62.675001)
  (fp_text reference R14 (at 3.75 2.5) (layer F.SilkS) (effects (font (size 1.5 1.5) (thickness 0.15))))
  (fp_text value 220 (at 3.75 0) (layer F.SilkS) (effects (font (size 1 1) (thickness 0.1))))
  (pad 1 thru_hole circle (at 0 0) (size 1.8 1.8) (drill 0.8) (layers *.Cu *.Mask F.SilkS) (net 11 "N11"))
  (pad 2 thru_hole circle (at 7.5 0) (size 1.8 1.8) (drill 0.8) (layers *.Cu *.Mask F.SilkS) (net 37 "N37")))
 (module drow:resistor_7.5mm (layer F.Cu) (at 34 63.5 180)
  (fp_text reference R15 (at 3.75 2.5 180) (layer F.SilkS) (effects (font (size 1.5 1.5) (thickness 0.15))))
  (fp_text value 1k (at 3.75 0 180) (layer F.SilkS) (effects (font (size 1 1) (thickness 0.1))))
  (pad 1 thru_hole circle (at 0 0 180) (size 1.8 1.8) (drill 0.8) (layers *.Cu *.Mask F.SilkS) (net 25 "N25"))
  (pad 2 thru_hole circle (at 7.5 0 180) (size 1.8 1.8) (drill 0.8) (layers *.Cu *.Mask F.SilkS) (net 33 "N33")))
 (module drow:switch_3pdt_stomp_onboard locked (layer F.Cu) (at 43.7 106.25)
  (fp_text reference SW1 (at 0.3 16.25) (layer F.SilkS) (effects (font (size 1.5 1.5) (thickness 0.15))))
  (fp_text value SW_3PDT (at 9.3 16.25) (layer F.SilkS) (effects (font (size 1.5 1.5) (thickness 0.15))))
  (pad 1 thru_hole circle (at 0 0) (size 3.2 3.2) (drill 1.5) (layers *.Cu *.Mask F.SilkS) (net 32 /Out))
  (pad 4 thru_hole circle (at 5.3 0) (size 3.2 3.2) (drill 1.5) (layers *.Cu *.Mask F.SilkS) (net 28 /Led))
  (pad 7 thru_hole circle (at 10.6 0) (size 3.2 3.2) (drill 1.5) (layers *.Cu *.Mask F.SilkS) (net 34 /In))
  (pad 6 thru_hole circle (at 5.3 4.7) (size 3.2 3.2) (drill 1.5) (layers *.Cu *.Mask F.SilkS) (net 6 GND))
  (pad 9 thru_hole circle (at 10.6 4.7) (size 3.2 3.2) (drill 1.5) (layers *.Cu *.Mask F.SilkS) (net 15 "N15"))
  (pad 2 thru_hole circle (at 0 9.4) (size 3.2 3.2) (drill 1.5) (layers *.Cu *.Mask F.SilkS) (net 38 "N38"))
  (pad 3 thru_hole circle (at 0 4.7) (size 3.2 3.2) (drill 1.5) (layers *.Cu *.Mask F.SilkS) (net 16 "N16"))
  (pad 5 thru_hole circle (at 5.3 9.4) (size 3.2 3.2) (drill 1.5) (layers *.Cu *.Mask F.SilkS) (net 34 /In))
  (pad 8 thru_hole circle (at 10.6 9.4) (size 3.2 3.2) (drill 1.5) (layers *.Cu *.Mask F.SilkS) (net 38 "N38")))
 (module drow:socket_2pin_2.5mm (layer F.Cu) (at 125.653572 72.875)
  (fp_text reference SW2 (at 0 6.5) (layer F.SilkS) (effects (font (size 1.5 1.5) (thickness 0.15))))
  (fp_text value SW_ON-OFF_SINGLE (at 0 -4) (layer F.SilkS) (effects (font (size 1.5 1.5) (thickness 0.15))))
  (pad 1 thru_hole oval (at 0 0) (size 3.5 2) (drill 1) (layers *.Cu *.Mask F.SilkS) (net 24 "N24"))
  (pad 2 thru_hole oval (at 0 2.5) (size 3.5 2) (drill 1) (layers *.Cu *.Mask F.SilkS) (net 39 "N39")))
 (gr_line (start 21 32) (end 21 123.5) (angle 90) (layer Edge.Cuts) (width 0.1))
 (gr_line (start 32 21) (end 21 32) (angle 90) (layer Edge.Cuts) (width 0.1))
 (gr_line (start 66 21) (end 32 21) (angle 90) (layer Edge.Cuts) (width 0.1))
 (gr_line (start 77 32) (end 66 21) (angle 90) (layer Edge.Cuts) (width 0.1))
 (gr_line (start 77 123.5) (end 77 32) (angle 90) (layer Edge.Cuts) (width 0.1))
 (gr_line (start 21 123.5) (end 77 123.5) (angle 90) (layer Edge.Cuts) (width 0.1))
 (segment (start 62.5 110.5) (end 62.5 108.5) (width 0.8) (layer B.Cu) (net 1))
 (segment (start 64.15 103.6) (end 62.5 105.25) (width 0.8) (layer B.Cu) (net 1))
 (segment (start 62.5 105.25) (end 62.5 108.5) (width 0.8) (layer B.Cu) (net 1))
 (segment (start 64.15 83.5) (end 64.15 100) (width 0.8) (layer B.Cu) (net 1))
 (segment (start 63 111) (end 62.5 110.5) (width 0.8) (layer B.Cu) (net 1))
 (segment (start 64.15 103.6) (end 64.15 100) (width 0.8) (layer B.Cu) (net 1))
 (segment (start 64.4 111) (end 63 111) (width 0.8) (layer B.Cu) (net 1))
 (segment (start 66.5 118.5) (end 66.5 114.6) (width 0.6) (layer B.Cu) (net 2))
 (segment (start 66.5 114.6) (end 70.1 111) (width 0.6) (layer B.Cu) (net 2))
 (segment (start 51.5 78.5) (end 51.5 76) (width 0.6) (layer B.Cu) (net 17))
 (segment (start 46.5 71) (end 44 71) (width 0.6) (layer B.Cu) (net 18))
 (segment (start 46.5 76) (end 46.5 71) (width 0.6) (layer B.Cu) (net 18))
 (segment (start 46.5 71) (end 49 68.5) (width 0.6) (layer B.Cu) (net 18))
 (segment (start 61.5 58.5) (end 56.5 63.5) (width 0.6) (layer B.Cu) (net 18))
 (segment (start 56.5 63.5) (end 51.5 63.5) (width 0.6) (layer B.Cu) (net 18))
 (segment (start 51.5 63.5) (end 49 66) (width 0.6) (layer B.Cu) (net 18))
 (segment (start 49 66) (end 49 68.5) (width 0.6) (layer B.Cu) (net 18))
 (segment (start 51.5 61) (end 49 61) (width 0.6) (layer B.Cu) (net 19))
 (segment (start 49 61) (end 46.5 63.5) (width 0.6) (layer B.Cu) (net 19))
 (segment (start 51.5 61) (end 54 58.5) (width 0.6) (layer B.Cu) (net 19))
 (segment (start 44 68.5) (end 36.5 68.5) (width 0.6) (layer B.Cu) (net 19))
 (segment (start 44 68.5) (end 46.5 66) (width 0.6) (layer B.Cu) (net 19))
 (segment (start 46.5 66) (end 46.5 63.5) (width 0.6) (layer B.Cu) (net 19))
 (segment (start 44 66) (end 41.5 63.5) (width 0.6) (layer B.Cu) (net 20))
 (segment (start 39 63.5) (end 41.5 63.5) (width 0.6) (layer B.Cu) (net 20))
 (segment (start 49 58.5) (end 44 58.5) (width 0.6) (layer B.Cu) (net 20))
 (segment (start 44 58.5) (end 44 61) (width 0.6) (layer B.Cu) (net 20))
 (segment (start 44 61) (end 41.5 63.5) (width 0.6) (layer B.Cu) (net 20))
 (segment (start 61.5 78.5) (end 62.55 79.55) (width 0.8) (layer B.Cu) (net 6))
 (segment (start 62.55 79.55) (end 62.55 80.5) (width 0.8) (layer B.Cu) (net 6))
 (segment (start 66.5 71) (end 66.5 80.5) (width 0.8) (layer B.Cu) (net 6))
 (segment (start 27.5 100) (end 33.85 100) (width 0.8) (layer B.Cu) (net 6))
 (segment (start 27.5 83.5) (end 27.5 100) (width 0.8) (layer B.Cu) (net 6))
 (segment (start 40.2 83.5) (end 27.5 83.5) (width 0.8) (layer B.Cu) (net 6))
 (segment (start 36.25 115.75) (end 41.5 121) (width 0.8) (layer B.Cu) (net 6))
 (segment (start 41.5 121) (end 56.5 121) (width 0.8) (layer B.Cu) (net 6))
 (segment (start 56.5 121) (end 60.3 117.2) (width 0.8) (layer B.Cu) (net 6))
 (segment (start 60.3 117.2) (end 60.3 102.5) (width 0.8) (layer B.Cu) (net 6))
 (segment (start 60.3 102.5) (end 57.8 100) (width 0.8) (layer B.Cu) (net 6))
 (segment (start 33.85 113.35) (end 36.25 115.75) (width 0.8) (layer B.Cu) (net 6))
 (segment (start 33.85 100) (end 33.85 113.35) (width 0.8) (layer B.Cu) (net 6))
 (segment (start 46.65 113.3) (end 38.7 113.3) (width 0.6) (layer B.Cu) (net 6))
 (segment (start 49 110.95) (end 46.65 113.3) (width 0.6) (layer B.Cu) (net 6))
 (segment (start 38.7 113.3) (end 36.25 115.75) (width 0.6) (layer B.Cu) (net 6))
 (segment (start 60.975 96.825) (end 57.8 100) (width 0.8) (layer B.Cu) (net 6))
 (segment (start 60.975 82.075) (end 60.975 96.825) (width 0.8) (layer B.Cu) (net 6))
 (segment (start 62.55 80.5) (end 60.975 82.075) (width 0.8) (layer B.Cu) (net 6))
 (segment (start 67.5 80.5) (end 66.5 80.5) (width 0.8) (layer B.Cu) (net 6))
 (segment (start 66.5 80.5) (end 62.55 80.5) (width 0.8) (layer B.Cu) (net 6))
 (segment (start 70.5 83.5) (end 67.5 80.5) (width 0.8) (layer B.Cu) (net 6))
 (segment (start 70.5 100) (end 70.5 83.5) (width 0.8) (layer B.Cu) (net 6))
 (segment (start 70 76) (end 71.5 74.5) (width 0.6) (layer B.Cu) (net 14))
 (segment (start 71.5 74.5) (end 71.5 71) (width 0.6) (layer B.Cu) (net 14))
 (segment (start 71.65 103.6) (end 74 101.25) (width 0.6) (layer B.Cu) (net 14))
 (segment (start 74 80) (end 70 76) (width 0.6) (layer B.Cu) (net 14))
 (segment (start 74 101.25) (end 74 80) (width 0.6) (layer B.Cu) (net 14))
 (segment (start 71.5 118.5) (end 73 117) (width 0.6) (layer B.Cu) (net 14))
 (segment (start 73 104.95) (end 71.65 103.6) (width 0.6) (layer B.Cu) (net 14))
 (segment (start 73 117) (end 73 104.95) (width 0.6) (layer B.Cu) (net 14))
 (segment (start 36.5 63.5) (end 34 63.5) (width 0.6) (layer B.Cu) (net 25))
 (segment (start 56.55 110.95) (end 57.8 109.7) (width 0.6) (layer B.Cu) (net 15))
 (segment (start 57.8 109.7) (end 57.8 104.55) (width 0.6) (layer B.Cu) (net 15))
 (segment (start 57.8 104.55) (end 54.25 101) (width 0.6) (layer B.Cu) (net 15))
 (segment (start 54.25 101) (end 54.25 87) (width 0.6) (layer B.Cu) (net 15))
 (segment (start 54.25 87) (end 57.8 83.5) (width 0.6) (layer B.Cu) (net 15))
 (segment (start 54.3 110.95) (end 56.55 110.95) (width 0.6) (layer B.Cu) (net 15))
 (segment (start 40.2 109.9) (end 41.25 110.95) (width 0.6) (layer B.Cu) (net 16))
 (segment (start 41.25 110.95) (end 43.65 110.95) (width 0.6) (layer B.Cu) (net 16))
 (segment (start 40.2 100) (end 40.2 109.9) (width 0.6) (layer B.Cu) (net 16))
 (segment (start 43.7 106.25) (end 46.5 103.45) (width 0.6) (layer B.Cu) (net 32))
 (segment (start 31.5 66) (end 31.5 68.5) (width 0.6) (layer B.Cu) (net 32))
 (segment (start 31.5 68.5) (end 44 81) (width 0.6) (layer B.Cu) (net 32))
 (segment (start 31.5 66) (end 31.5 58.5) (width 0.6) (layer B.Cu) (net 32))
 (segment (start 46.5 83.5) (end 44 81) (width 0.6) (layer B.Cu) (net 32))
 (segment (start 46.5 103.45) (end 46.5 83.5) (width 0.6) (layer B.Cu) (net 32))
 (segment (start 26.5 63.5) (end 26.5 58.5) (width 0.6) (layer B.Cu) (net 33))
 (segment (start 54.3 106.25) (end 51.5 103.45) (width 0.6) (layer B.Cu) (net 34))
 (segment (start 54 81) (end 54 78.5) (width 0.6) (layer B.Cu) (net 34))
 (segment (start 51.5 83.5) (end 54 81) (width 0.6) (layer B.Cu) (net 34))
 (segment (start 51.5 103.45) (end 51.5 83.5) (width 0.6) (layer B.Cu) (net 34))
 (segment (start 51.65 113) (end 51.65 108.9) (width 0.6) (layer B.Cu) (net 34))
 (segment (start 51.65 108.9) (end 54.3 106.25) (width 0.6) (layer B.Cu) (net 34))
 (segment (start 49 115.65) (end 51.65 113) (width 0.6) (layer B.Cu) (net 34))
 (segment (start 46.55 118.5) (end 51.45 118.5) (width 0.6) (layer B.Cu) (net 38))
 (segment (start 51.45 118.5) (end 54.3 115.65) (width 0.6) (layer B.Cu) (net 38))
 (segment (start 43.7 115.65) (end 46.55 118.5) (width 0.6) (layer B.Cu) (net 38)))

